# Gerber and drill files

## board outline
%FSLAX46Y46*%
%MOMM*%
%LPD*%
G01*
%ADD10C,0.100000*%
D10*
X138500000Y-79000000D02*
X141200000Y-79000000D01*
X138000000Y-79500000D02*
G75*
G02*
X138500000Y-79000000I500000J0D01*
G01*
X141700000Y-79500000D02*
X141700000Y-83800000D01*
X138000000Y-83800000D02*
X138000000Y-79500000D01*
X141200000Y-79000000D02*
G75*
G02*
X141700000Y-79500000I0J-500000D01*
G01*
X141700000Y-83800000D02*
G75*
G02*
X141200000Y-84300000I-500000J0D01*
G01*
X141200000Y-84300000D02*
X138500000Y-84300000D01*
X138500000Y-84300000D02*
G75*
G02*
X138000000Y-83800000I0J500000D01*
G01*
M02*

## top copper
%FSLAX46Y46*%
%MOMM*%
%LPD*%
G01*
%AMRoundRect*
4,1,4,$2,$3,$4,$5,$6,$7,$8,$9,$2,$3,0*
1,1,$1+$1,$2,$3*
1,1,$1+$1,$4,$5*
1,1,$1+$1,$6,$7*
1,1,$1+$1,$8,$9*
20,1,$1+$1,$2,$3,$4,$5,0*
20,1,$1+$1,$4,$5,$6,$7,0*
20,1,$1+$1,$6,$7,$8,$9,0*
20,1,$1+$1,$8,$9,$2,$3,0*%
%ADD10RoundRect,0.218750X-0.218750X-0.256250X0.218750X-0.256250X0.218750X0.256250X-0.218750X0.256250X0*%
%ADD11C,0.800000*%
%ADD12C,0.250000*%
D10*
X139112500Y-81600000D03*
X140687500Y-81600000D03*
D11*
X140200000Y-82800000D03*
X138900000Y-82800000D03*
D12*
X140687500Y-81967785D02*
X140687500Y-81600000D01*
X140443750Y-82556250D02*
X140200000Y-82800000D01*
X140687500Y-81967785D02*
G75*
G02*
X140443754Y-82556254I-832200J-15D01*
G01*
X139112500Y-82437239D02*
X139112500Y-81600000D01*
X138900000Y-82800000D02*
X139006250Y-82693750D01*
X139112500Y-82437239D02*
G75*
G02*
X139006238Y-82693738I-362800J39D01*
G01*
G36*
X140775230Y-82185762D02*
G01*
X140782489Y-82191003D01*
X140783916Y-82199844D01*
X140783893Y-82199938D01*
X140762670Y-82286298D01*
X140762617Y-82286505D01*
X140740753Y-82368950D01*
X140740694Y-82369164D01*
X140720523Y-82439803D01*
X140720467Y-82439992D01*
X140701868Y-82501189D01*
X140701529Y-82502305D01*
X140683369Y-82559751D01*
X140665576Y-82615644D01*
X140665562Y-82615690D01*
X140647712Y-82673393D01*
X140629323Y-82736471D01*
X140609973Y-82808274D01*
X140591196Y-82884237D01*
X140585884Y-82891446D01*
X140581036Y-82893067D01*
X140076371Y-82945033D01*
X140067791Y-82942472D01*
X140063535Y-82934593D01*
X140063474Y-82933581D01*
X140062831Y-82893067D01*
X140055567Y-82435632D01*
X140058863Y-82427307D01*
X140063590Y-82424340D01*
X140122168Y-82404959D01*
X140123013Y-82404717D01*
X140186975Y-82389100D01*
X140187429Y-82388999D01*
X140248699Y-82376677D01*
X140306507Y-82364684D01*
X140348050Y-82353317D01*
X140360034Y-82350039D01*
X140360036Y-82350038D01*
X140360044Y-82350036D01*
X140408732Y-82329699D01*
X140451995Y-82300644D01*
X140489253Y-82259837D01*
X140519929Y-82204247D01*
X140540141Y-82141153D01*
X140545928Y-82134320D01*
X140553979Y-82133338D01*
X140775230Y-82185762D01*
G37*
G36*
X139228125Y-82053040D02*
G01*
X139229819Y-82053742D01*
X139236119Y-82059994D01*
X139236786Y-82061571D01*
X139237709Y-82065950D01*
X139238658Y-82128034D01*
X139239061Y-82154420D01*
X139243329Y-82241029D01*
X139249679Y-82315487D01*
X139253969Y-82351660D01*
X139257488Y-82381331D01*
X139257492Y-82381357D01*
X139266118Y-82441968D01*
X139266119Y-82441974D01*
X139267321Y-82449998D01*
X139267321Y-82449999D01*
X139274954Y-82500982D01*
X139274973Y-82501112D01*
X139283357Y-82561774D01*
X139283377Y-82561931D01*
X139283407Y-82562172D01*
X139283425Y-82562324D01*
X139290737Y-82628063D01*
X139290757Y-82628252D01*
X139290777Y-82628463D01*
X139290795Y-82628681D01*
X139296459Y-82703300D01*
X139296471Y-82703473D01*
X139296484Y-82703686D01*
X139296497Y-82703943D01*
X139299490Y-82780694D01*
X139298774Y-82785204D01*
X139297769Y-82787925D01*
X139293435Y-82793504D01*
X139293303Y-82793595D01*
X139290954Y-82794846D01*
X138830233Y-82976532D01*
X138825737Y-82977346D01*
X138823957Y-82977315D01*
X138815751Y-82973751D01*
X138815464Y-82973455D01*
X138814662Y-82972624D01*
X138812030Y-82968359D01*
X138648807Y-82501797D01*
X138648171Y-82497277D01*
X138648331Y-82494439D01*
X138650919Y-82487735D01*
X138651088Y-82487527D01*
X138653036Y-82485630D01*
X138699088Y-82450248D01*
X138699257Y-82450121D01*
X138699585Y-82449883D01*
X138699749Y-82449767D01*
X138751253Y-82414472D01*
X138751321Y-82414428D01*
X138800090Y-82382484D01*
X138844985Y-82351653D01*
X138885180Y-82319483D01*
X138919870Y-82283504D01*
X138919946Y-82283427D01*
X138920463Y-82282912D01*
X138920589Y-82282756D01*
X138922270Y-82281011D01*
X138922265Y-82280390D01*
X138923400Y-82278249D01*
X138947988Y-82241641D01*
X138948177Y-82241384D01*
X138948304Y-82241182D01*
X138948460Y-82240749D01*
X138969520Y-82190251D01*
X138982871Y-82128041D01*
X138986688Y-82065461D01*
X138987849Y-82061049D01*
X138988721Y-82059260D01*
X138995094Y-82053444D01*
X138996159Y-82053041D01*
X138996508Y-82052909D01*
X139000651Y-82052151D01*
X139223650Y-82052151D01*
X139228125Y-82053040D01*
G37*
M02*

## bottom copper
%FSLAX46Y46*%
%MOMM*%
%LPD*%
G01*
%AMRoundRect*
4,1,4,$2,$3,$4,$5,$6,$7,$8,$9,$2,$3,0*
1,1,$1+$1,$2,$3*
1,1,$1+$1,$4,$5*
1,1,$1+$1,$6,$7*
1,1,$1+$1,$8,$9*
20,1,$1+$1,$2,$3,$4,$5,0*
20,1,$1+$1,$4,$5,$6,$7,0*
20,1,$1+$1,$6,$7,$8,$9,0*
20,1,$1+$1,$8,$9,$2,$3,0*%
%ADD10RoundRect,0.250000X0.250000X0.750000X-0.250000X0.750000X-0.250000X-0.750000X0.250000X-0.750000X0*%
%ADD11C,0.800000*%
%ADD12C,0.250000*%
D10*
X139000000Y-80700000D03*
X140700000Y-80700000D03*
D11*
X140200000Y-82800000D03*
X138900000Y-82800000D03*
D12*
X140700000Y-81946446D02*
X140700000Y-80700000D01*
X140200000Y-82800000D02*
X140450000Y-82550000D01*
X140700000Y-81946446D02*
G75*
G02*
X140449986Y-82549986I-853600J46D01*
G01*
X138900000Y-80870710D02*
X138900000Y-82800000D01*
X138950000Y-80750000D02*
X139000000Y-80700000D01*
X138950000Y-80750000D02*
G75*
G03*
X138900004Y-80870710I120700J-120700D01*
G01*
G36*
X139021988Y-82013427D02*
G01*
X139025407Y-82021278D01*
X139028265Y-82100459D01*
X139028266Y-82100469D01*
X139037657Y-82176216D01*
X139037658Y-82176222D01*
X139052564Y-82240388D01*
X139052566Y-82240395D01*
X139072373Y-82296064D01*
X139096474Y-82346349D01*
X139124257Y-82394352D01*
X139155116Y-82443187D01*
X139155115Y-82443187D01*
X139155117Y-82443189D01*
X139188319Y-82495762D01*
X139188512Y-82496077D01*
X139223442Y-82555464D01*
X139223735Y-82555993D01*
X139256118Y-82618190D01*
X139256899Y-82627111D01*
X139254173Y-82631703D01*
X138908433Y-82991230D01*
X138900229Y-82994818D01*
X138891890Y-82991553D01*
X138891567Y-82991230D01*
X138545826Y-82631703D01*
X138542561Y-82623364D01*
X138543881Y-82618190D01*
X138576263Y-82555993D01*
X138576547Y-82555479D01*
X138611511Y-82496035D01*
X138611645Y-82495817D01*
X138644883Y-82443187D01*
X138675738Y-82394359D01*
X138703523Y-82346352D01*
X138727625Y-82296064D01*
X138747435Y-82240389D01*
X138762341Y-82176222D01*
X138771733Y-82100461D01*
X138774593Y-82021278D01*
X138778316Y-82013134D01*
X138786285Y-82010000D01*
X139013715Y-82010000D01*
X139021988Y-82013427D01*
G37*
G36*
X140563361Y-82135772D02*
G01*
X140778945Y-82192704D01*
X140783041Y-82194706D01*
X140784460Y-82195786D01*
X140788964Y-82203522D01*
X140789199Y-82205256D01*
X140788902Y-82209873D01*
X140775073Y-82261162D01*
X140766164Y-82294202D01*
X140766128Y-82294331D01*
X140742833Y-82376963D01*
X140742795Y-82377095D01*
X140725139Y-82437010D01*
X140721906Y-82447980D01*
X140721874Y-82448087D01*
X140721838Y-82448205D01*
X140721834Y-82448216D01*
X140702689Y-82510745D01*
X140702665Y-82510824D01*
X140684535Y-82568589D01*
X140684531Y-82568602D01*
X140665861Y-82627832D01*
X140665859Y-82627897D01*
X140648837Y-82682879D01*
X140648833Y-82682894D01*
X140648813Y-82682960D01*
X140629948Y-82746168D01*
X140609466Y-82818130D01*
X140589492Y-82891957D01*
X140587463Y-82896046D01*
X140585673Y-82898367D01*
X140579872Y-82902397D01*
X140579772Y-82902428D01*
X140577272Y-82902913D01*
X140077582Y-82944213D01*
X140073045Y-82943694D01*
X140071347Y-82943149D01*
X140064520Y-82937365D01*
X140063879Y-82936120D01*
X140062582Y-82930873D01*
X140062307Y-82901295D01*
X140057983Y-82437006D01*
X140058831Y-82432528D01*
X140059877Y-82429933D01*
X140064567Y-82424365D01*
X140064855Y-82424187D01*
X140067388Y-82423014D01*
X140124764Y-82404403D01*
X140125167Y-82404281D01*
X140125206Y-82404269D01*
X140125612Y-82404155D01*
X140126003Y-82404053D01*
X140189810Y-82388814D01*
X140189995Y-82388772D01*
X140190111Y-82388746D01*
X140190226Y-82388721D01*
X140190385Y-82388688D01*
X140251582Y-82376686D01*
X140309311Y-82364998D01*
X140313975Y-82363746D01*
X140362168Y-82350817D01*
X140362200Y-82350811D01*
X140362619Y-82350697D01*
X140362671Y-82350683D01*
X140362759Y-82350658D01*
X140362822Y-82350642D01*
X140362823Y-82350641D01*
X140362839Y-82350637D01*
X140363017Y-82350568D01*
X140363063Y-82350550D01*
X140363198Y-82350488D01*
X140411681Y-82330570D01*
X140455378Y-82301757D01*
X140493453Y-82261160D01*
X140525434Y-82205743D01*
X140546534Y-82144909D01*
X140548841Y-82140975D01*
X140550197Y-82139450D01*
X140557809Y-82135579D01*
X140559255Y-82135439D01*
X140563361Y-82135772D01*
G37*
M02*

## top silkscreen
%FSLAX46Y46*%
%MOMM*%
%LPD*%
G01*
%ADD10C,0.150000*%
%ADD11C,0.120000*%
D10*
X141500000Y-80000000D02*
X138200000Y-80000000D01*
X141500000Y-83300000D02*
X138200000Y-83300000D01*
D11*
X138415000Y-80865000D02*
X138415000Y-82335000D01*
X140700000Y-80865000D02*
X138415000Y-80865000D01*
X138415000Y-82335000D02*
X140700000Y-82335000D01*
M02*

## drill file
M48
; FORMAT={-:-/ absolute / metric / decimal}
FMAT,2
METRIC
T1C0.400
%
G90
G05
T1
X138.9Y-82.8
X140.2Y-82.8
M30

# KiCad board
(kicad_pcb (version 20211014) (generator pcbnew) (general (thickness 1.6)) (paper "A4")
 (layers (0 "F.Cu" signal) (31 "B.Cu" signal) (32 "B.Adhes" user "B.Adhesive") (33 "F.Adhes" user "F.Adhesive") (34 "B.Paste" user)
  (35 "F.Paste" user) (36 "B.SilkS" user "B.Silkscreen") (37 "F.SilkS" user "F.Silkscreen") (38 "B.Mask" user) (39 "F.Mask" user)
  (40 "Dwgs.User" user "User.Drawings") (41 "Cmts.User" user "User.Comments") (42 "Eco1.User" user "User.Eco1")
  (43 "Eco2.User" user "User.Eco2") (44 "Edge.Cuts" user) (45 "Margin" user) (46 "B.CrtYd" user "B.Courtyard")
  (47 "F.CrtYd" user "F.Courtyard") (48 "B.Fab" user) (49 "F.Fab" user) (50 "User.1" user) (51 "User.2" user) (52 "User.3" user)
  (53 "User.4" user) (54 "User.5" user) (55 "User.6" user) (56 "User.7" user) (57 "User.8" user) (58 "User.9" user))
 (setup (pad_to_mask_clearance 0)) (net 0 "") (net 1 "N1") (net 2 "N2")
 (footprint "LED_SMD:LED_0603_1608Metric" (layer "F.Cu") (at 139.9 81.6)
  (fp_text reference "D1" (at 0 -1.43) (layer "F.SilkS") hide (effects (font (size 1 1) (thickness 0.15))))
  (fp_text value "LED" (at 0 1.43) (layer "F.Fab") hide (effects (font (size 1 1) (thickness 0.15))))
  (fp_line (start -1.485 -0.735) (end -1.485 0.735) (layer "F.SilkS") (width 0.12))
  (fp_line (start 0.8 -0.735) (end -1.485 -0.735) (layer "F.SilkS") (width 0.12))
  (fp_line (start -1.485 0.735) (end 0.8 0.735) (layer "F.SilkS") (width 0.12))
  (pad "1" smd roundrect (at -0.7875 0) (size 0.875 0.95) (layers "F.Cu" "F.Paste" "F.Mask") (roundrect_rratio 0.25) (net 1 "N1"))
  (pad "2" smd roundrect (at 0.7875 0) (size 0.875 0.95) (layers "F.Cu" "F.Paste" "F.Mask") (roundrect_rratio 0.25) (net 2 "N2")))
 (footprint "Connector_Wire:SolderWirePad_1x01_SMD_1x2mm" (layer "B.Cu") (at 139 80.7 180)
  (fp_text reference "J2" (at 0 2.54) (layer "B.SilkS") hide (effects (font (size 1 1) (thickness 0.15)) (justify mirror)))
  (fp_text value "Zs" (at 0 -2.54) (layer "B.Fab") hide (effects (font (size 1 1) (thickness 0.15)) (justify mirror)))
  (pad "1" smd roundrect (at 0 0 180) (size 1 2) (layers "B.Cu" "B.Paste" "B.Mask") (roundrect_rratio 0.25) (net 1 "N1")))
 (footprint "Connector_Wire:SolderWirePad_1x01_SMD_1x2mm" (layer "B.Cu") (at 140.7 80.7 180)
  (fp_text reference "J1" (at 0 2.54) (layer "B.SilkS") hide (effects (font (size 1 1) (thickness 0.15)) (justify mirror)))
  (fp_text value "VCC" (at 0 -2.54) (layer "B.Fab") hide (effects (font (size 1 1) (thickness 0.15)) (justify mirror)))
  (pad "1" smd roundrect (at 0 0 180) (size 1 2) (layers "B.Cu" "B.Paste" "B.Mask") (roundrect_rratio 0.25) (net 2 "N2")))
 (gr_line (start 141.5 80) (end 138.2 80) (layer "F.SilkS") (width 0.15))
 (gr_line (start 141.5 83.3) (end 138.2 83.3) (layer "F.SilkS") (width 0.15))
 (gr_line (start 138.5 79) (end 141.2 79) (layer "Edge.Cuts") (width 0.1))
 (gr_arc (start 138 79.5) (mid 138.146447 79.146447) (end 138.5 79) (layer "Edge.Cuts") (width 0.1))
 (gr_line (start 141.7 79.5) (end 141.7 83.8) (layer "Edge.Cuts") (width 0.1))
 (gr_line (start 138 83.8) (end 138 79.5) (layer "Edge.Cuts") (width 0.1))
 (gr_arc (start 141.2 79) (mid 141.553553 79.146447) (end 141.7 79.5) (layer "Edge.Cuts") (width 0.1))
 (gr_arc (start 141.7 83.8) (mid 141.553553 84.153553) (end 141.2 84.3) (layer "Edge.Cuts") (width 0.1))
 (gr_line (start 141.2 84.3) (end 138.5 84.3) (layer "Edge.Cuts") (width 0.1))
 (gr_arc (start 138.5 84.3) (mid 138.146447 84.153553) (end 138 83.8) (layer "Edge.Cuts") (width 0.1))
 (segment (start 140.6875 81.967785) (end 140.6875 81.6) (width 0.25) (layer "F.Cu") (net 2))
 (segment (start 140.44375 82.55625) (end 140.2 82.8) (width 0.25) (layer "F.Cu") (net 2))
 (via (at 140.2 82.8) (size 0.8) (drill 0.4) (layers "F.Cu" "B.Cu") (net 2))
 (arc (start 140.6875 81.967785) (mid 140.624151 82.28626) (end 140.44375 82.55625) (width 0.25) (layer "F.Cu") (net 2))
 (segment (start 140.7 81.946446) (end 140.7 80.7) (width 0.25) (layer "B.Cu") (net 2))
 (segment (start 140.2 82.8) (end 140.45 82.55) (width 0.25) (layer "B.Cu") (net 2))
 (arc (start 140.7 81.946446) (mid 140.635027 82.273087) (end 140.45 82.55) (width 0.25) (layer "B.Cu") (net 2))
 (segment (start 139.1125 82.437239) (end 139.1125 81.6) (width 0.25) (layer "F.Cu") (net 1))
 (segment (start 138.9 82.8) (end 139.00625 82.69375) (width 0.25) (layer "F.Cu") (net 1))
 (via (at 138.9 82.8) (size 0.8) (drill 0.4) (layers "F.Cu" "B.Cu") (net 1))
 (arc (start 139.1125 82.437239) (mid 139.084886 82.576061) (end 139.00625 82.69375) (width 0.25) (layer "F.Cu") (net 1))
 (segment (start 138.9 80.87071) (end 138.9 82.8) (width 0.25) (layer "B.Cu") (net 1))
 (segment (start 138.95 80.75) (end 139 80.7) (width 0.25) (layer "B.Cu") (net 1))
 (arc (start 138.95 80.75) (mid 138.912994 80.805382) (end 138.9 80.87071) (width 0.25) (layer "B.Cu") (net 1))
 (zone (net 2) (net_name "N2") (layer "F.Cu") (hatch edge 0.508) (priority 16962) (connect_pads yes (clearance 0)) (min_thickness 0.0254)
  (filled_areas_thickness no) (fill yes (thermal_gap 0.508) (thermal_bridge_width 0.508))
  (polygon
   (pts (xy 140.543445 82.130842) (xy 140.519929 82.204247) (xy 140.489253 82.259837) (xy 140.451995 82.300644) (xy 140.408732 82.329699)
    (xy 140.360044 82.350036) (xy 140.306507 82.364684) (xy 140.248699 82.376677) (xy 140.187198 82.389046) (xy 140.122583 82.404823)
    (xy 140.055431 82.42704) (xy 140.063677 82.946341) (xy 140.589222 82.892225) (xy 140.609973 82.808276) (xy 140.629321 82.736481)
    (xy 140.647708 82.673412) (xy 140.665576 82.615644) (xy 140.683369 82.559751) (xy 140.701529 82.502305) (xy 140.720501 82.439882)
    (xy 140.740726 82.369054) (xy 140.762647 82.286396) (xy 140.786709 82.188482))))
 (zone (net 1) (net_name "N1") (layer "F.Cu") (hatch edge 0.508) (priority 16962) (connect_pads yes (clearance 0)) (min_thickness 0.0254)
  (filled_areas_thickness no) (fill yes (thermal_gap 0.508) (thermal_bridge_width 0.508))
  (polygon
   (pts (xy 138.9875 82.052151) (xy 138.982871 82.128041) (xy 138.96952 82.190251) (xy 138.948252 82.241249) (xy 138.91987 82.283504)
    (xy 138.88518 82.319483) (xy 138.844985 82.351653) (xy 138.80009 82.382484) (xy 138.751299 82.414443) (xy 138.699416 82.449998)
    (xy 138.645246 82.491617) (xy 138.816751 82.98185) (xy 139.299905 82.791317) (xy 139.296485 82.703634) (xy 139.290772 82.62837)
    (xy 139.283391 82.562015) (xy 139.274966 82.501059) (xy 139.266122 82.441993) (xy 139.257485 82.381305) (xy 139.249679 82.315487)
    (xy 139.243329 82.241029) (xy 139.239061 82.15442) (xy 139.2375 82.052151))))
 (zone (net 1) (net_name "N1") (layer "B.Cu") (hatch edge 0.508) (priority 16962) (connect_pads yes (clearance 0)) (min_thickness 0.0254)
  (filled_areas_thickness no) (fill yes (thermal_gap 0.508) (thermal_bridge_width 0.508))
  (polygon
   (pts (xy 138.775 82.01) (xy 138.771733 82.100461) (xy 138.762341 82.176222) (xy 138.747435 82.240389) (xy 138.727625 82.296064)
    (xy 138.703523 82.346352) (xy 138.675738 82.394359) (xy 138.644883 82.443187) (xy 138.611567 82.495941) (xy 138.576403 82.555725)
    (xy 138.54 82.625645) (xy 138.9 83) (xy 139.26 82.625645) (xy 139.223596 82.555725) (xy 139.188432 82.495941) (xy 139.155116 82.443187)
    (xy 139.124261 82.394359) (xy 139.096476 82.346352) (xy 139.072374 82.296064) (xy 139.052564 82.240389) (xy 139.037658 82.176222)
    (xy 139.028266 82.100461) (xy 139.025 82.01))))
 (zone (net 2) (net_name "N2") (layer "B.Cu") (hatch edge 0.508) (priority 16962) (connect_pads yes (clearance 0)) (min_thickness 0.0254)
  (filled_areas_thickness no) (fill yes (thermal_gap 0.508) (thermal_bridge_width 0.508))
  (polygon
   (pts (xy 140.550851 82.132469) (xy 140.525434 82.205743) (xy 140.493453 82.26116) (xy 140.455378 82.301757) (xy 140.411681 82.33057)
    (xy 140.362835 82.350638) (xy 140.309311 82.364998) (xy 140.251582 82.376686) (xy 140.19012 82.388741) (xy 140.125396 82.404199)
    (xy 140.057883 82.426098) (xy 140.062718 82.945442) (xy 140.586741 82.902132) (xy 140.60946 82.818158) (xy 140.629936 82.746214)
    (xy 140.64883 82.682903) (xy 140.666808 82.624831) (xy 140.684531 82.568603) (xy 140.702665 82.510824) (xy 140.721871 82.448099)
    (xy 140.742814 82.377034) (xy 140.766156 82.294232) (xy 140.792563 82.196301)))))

